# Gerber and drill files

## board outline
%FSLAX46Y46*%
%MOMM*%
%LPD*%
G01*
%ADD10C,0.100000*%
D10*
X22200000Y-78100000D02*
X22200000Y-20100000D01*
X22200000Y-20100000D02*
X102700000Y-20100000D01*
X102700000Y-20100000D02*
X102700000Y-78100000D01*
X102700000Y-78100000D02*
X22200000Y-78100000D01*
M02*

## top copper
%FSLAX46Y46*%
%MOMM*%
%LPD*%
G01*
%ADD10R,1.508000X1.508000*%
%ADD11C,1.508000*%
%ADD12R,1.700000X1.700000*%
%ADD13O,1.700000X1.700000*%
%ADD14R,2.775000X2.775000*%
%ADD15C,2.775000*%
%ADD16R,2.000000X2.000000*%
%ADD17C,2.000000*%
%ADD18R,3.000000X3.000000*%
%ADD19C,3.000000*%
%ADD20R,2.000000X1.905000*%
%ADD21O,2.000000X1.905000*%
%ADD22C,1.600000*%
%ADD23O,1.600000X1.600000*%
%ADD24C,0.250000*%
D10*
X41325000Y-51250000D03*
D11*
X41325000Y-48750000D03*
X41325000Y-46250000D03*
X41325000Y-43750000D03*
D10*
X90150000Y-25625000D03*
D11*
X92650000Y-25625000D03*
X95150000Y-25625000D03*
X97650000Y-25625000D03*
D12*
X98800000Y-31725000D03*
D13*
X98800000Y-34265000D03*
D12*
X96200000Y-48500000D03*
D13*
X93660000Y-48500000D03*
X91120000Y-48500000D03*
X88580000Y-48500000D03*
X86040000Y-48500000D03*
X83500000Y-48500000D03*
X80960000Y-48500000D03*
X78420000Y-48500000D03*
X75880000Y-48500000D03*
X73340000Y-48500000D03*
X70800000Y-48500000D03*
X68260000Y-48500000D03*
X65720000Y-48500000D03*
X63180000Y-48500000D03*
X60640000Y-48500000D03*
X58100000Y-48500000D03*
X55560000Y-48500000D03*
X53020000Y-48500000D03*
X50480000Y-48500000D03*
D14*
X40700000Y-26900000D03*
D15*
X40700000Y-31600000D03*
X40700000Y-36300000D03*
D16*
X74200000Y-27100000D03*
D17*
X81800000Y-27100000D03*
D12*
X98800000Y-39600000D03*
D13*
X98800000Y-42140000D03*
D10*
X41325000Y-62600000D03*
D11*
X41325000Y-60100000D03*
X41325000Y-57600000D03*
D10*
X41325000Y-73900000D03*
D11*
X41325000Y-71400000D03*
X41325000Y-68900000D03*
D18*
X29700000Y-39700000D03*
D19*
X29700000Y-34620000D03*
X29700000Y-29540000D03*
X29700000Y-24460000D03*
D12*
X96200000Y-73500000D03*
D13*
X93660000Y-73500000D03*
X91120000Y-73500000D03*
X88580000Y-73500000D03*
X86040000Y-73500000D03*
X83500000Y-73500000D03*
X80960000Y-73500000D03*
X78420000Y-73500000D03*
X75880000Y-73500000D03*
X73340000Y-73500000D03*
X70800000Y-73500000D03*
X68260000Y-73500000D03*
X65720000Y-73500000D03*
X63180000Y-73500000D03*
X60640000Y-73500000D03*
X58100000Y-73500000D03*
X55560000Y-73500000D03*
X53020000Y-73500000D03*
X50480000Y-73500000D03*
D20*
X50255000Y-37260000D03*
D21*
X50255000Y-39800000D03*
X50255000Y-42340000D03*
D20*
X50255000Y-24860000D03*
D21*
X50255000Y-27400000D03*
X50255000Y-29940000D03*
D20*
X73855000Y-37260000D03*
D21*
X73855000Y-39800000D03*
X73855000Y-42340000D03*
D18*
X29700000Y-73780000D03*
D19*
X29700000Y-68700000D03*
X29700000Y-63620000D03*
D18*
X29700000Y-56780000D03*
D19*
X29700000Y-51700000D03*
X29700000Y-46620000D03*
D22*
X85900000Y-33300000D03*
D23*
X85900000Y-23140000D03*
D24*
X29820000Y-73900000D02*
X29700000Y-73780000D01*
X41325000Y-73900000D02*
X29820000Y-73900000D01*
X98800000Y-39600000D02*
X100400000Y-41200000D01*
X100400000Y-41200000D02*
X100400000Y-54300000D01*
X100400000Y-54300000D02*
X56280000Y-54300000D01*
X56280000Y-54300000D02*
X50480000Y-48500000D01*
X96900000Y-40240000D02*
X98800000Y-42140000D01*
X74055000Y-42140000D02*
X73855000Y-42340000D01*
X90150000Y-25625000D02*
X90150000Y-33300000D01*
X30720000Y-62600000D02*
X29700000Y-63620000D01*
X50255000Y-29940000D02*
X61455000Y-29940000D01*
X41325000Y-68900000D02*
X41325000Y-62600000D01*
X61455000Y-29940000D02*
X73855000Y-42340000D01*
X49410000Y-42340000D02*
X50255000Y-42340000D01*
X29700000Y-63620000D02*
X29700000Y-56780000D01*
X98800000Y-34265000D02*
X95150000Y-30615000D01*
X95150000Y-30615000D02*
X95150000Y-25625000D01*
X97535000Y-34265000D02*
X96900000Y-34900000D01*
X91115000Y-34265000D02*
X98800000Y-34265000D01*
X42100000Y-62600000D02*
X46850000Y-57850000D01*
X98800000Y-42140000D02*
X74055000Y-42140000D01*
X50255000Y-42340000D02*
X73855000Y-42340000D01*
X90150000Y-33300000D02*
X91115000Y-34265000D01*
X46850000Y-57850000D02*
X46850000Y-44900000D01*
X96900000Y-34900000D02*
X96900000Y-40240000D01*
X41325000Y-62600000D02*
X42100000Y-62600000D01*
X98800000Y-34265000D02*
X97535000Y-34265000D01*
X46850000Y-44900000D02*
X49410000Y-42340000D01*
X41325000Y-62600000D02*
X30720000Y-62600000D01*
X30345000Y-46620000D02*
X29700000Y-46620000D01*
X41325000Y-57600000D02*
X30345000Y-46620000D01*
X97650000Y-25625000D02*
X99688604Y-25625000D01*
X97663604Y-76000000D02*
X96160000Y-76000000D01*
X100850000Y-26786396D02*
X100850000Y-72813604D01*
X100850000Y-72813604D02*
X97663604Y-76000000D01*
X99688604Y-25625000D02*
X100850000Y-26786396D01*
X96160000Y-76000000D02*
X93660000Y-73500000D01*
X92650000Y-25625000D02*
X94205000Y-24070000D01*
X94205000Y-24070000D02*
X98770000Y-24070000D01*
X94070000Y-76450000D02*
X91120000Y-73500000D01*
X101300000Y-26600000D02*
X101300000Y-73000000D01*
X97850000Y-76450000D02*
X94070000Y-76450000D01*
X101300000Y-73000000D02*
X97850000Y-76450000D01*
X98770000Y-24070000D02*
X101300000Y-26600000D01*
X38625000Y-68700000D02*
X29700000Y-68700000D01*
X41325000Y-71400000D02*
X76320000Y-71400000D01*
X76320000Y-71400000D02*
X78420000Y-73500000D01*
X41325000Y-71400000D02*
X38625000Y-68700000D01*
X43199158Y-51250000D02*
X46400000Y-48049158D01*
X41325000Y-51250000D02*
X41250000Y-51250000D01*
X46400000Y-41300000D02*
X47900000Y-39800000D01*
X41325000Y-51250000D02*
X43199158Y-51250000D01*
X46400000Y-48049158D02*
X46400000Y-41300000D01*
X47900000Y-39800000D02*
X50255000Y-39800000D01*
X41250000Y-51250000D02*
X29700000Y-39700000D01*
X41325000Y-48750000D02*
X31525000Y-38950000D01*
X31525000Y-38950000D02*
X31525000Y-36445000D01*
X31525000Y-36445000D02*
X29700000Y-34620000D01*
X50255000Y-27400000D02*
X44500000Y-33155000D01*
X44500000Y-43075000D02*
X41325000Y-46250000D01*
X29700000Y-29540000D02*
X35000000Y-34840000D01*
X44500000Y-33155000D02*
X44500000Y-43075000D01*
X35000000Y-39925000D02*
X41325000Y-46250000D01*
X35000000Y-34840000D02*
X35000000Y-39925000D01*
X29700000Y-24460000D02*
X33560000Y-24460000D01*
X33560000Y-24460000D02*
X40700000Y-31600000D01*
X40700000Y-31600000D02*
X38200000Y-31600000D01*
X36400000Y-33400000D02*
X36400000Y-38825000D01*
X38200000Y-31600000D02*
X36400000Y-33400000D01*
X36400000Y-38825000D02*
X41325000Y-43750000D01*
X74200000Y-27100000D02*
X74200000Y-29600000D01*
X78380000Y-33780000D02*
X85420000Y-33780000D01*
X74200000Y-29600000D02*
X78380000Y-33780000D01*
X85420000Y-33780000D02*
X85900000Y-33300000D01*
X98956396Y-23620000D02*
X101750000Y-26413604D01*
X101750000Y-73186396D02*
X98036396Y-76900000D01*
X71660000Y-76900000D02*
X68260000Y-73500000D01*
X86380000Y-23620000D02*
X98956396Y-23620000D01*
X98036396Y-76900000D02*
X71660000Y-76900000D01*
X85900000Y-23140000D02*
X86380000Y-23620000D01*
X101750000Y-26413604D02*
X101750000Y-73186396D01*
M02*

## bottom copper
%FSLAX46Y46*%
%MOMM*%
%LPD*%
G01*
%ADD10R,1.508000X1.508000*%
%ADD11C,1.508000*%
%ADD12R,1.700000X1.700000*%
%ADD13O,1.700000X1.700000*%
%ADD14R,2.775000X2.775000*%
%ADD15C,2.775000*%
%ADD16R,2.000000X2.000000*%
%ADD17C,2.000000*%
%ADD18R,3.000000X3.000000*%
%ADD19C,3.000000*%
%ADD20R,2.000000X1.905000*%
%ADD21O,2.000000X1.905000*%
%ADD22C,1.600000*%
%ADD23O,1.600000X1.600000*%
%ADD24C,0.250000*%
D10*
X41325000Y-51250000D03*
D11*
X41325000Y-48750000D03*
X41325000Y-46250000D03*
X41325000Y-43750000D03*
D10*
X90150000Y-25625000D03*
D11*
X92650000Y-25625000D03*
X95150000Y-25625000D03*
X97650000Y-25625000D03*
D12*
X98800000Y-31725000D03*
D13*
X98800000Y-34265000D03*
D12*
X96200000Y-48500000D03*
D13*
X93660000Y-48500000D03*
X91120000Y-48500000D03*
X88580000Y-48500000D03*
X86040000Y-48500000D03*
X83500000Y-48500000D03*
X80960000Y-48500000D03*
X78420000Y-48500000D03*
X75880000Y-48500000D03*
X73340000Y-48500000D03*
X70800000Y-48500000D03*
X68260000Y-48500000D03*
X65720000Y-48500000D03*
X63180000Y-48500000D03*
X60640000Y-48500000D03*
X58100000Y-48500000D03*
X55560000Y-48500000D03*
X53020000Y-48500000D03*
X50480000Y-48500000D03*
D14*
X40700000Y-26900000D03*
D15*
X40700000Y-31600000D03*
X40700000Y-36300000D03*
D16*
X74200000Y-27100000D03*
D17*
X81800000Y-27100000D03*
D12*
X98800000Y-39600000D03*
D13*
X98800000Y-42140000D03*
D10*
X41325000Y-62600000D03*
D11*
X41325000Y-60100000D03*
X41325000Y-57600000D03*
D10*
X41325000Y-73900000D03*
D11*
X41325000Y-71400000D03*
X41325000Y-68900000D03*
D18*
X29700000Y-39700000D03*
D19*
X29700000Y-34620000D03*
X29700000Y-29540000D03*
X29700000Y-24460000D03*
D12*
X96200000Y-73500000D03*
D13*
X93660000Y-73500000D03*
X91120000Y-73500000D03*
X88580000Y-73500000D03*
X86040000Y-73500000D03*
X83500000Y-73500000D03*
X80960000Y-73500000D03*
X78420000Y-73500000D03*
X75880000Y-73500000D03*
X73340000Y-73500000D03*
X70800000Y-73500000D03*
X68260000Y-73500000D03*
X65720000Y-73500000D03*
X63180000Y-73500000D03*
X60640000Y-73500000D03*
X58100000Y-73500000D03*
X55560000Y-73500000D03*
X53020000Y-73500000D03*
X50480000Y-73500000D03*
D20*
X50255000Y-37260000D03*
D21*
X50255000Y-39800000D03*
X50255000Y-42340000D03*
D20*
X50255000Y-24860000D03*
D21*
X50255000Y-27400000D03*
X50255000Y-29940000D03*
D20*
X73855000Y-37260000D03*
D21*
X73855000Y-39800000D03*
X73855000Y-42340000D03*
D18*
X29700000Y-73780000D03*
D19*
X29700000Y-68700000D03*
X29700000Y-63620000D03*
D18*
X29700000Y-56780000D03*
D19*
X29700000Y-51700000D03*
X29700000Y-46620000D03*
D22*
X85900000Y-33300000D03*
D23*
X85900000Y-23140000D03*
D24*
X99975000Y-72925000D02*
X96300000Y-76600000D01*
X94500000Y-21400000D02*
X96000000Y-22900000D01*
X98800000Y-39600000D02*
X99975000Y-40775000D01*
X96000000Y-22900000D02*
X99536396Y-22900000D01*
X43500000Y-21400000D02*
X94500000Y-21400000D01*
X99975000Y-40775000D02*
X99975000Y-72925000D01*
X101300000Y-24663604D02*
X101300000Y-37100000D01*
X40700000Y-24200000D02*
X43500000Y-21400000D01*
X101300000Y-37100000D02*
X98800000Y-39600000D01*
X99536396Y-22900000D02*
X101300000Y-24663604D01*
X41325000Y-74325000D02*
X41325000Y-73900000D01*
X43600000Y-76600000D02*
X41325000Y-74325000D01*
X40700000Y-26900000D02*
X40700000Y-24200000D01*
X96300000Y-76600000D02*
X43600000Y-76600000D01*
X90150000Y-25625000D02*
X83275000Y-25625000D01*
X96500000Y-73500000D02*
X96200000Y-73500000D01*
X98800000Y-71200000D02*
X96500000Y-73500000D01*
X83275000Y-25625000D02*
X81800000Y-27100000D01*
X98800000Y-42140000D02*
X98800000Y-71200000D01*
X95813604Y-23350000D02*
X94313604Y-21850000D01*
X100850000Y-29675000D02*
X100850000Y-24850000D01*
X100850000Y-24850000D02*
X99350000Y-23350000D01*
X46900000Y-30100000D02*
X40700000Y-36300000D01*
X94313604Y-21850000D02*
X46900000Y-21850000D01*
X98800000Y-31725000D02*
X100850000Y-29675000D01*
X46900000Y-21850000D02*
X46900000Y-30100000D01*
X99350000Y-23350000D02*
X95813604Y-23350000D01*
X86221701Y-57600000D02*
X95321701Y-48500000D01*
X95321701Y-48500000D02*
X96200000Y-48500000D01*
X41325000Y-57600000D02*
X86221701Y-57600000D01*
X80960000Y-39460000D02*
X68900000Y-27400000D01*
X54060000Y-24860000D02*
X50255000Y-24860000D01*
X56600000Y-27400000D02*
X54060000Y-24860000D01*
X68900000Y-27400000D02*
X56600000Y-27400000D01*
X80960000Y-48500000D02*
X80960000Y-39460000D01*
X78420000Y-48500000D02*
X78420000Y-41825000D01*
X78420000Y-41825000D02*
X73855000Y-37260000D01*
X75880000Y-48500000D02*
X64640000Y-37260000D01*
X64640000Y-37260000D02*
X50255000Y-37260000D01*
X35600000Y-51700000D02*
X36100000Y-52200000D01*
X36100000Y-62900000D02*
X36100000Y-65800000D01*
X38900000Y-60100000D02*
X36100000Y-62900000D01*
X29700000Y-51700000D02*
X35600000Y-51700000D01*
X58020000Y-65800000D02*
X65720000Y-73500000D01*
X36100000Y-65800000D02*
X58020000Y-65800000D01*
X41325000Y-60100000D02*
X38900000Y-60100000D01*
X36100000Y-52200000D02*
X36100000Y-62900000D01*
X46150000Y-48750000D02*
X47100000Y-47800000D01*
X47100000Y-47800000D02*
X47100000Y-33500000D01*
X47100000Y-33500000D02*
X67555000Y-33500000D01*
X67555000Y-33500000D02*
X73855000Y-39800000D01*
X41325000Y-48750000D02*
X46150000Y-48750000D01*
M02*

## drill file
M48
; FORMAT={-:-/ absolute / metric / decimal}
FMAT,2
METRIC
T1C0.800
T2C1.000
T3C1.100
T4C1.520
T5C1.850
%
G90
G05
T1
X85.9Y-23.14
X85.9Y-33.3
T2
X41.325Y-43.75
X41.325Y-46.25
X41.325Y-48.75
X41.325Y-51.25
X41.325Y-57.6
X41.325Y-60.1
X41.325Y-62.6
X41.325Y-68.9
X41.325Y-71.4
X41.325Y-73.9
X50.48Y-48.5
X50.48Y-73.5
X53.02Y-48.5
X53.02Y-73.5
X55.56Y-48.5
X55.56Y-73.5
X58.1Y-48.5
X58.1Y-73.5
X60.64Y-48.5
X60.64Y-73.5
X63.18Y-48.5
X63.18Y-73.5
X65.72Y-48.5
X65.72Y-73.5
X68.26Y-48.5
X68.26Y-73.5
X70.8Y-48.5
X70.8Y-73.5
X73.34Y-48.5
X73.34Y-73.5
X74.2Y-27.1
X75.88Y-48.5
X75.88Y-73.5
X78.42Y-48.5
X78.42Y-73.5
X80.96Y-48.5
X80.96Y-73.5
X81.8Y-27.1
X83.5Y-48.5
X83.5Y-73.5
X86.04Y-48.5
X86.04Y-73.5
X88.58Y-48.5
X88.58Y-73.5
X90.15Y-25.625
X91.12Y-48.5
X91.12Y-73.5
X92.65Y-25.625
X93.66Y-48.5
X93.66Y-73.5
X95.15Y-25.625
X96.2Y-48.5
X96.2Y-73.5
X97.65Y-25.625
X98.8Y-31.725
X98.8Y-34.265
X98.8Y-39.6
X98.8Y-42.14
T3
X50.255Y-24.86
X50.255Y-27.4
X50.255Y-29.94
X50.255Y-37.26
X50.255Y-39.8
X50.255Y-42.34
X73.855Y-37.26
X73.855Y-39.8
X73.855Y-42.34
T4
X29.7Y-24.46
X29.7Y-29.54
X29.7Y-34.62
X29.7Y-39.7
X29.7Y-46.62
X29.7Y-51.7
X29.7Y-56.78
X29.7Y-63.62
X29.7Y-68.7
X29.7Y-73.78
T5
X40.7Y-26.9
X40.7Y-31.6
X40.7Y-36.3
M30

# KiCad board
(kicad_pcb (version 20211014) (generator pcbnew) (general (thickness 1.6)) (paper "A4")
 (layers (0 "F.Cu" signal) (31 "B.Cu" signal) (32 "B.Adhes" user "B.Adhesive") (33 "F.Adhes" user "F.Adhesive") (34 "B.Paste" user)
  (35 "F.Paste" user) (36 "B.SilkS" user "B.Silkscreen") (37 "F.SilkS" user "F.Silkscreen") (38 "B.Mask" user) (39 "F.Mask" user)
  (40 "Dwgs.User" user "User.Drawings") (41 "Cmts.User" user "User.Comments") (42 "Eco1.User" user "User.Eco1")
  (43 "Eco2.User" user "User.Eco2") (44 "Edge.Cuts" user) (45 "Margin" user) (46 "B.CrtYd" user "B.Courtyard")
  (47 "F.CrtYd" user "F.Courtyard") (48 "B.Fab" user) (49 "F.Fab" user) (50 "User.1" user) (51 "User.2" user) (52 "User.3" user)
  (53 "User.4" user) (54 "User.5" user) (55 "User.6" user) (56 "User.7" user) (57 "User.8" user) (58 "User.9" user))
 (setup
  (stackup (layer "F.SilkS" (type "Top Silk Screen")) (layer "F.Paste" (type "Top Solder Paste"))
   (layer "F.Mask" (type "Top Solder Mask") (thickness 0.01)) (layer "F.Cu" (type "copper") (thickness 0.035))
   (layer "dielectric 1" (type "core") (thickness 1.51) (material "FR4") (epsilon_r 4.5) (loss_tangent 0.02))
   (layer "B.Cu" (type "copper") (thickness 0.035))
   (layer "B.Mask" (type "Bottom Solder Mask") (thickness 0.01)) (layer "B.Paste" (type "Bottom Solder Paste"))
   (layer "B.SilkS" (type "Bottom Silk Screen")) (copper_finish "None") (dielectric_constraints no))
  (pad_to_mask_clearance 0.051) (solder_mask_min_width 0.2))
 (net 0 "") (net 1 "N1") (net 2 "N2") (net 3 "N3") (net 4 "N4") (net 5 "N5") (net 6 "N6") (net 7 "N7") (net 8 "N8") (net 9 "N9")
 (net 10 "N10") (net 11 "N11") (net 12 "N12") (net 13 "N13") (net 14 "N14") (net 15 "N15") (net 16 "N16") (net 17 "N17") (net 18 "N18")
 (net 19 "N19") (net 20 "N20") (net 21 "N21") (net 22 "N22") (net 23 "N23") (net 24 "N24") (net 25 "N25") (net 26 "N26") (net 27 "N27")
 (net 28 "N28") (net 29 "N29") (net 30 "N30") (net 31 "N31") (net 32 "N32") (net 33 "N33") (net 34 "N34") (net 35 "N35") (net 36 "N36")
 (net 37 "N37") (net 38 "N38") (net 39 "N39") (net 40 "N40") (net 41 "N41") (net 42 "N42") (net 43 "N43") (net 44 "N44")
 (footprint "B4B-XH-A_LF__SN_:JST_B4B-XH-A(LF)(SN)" (layer "F.Cu") (at 40.8 47.5 90)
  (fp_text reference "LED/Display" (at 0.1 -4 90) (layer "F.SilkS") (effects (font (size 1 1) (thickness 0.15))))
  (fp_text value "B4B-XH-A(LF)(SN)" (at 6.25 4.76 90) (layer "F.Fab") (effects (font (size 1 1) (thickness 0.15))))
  (pad "1" thru_hole rect locked (at -3.75 0.525 90) (size 1.508 1.508) (drill 1) (layers *.Cu *.Mask) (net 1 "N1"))
  (pad "2" thru_hole circle locked (at -1.25 0.525 90) (size 1.508 1.508) (drill 1) (layers *.Cu *.Mask) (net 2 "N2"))
  (pad "3" thru_hole circle locked (at 1.25 0.525 90) (size 1.508 1.508) (drill 1) (layers *.Cu *.Mask) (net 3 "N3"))
  (pad "4" thru_hole circle locked (at 3.75 0.525 90) (size 1.508 1.508) (drill 1) (layers *.Cu *.Mask) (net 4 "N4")))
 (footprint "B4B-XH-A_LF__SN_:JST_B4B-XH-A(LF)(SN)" (layer "F.Cu") (at 93.9 25.1)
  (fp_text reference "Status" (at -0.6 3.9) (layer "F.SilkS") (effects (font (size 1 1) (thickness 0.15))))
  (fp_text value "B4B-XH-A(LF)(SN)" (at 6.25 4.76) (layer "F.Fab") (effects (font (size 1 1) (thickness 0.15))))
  (pad "1" thru_hole rect locked (at -3.75 0.525) (size 1.508 1.508) (drill 1) (layers *.Cu *.Mask) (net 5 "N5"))
  (pad "2" thru_hole circle locked (at -1.25 0.525) (size 1.508 1.508) (drill 1) (layers *.Cu *.Mask) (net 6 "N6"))
  (pad "3" thru_hole circle locked (at 1.25 0.525) (size 1.508 1.508) (drill 1) (layers *.Cu *.Mask) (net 5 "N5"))
  (pad "4" thru_hole circle locked (at 3.75 0.525) (size 1.508 1.508) (drill 1) (layers *.Cu *.Mask) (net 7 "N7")))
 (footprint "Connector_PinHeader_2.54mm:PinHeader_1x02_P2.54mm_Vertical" (layer "F.Cu") (at 98.8 31.725)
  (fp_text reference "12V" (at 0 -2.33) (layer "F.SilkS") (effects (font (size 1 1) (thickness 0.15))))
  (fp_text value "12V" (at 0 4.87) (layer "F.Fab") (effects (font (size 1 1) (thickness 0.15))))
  (pad "1" thru_hole rect (at 0 0) (size 1.7 1.7) (drill 1) (layers *.Cu *.Mask) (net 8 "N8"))
  (pad "2" thru_hole oval (at 0 2.54) (size 1.7 1.7) (drill 1) (layers *.Cu *.Mask) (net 5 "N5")))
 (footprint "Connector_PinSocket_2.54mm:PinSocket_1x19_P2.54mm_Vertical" (layer "F.Cu") (at 96.2 48.5 -90)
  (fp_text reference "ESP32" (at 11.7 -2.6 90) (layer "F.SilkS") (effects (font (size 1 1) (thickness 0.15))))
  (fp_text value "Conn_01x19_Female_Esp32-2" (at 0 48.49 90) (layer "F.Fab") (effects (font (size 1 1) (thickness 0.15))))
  (pad "1" thru_hole rect (at 0 0 270) (size 1.7 1.7) (drill 1) (layers *.Cu *.Mask) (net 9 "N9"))
  (pad "2" thru_hole oval (at 0 2.54 270) (size 1.7 1.7) (drill 1) (layers *.Cu *.Mask) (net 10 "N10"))
  (pad "3" thru_hole oval (at 0 5.08 270) (size 1.7 1.7) (drill 1) (layers *.Cu *.Mask) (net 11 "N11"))
  (pad "4" thru_hole oval (at 0 7.62 270) (size 1.7 1.7) (drill 1) (layers *.Cu *.Mask) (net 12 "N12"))
  (pad "5" thru_hole oval (at 0 10.16 270) (size 1.7 1.7) (drill 1) (layers *.Cu *.Mask) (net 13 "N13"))
  (pad "6" thru_hole oval (at 0 12.7 270) (size 1.7 1.7) (drill 1) (layers *.Cu *.Mask) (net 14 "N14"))
  (pad "7" thru_hole oval (at 0 15.24 270) (size 1.7 1.7) (drill 1) (layers *.Cu *.Mask) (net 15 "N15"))
  (pad "8" thru_hole oval (at 0 17.78 270) (size 1.7 1.7) (drill 1) (layers *.Cu *.Mask) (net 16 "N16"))
  (pad "9" thru_hole oval (at 0 20.32 270) (size 1.7 1.7) (drill 1) (layers *.Cu *.Mask) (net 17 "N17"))
  (pad "10" thru_hole oval (at 0 22.86 270) (size 1.7 1.7) (drill 1) (layers *.Cu *.Mask) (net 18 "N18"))
  (pad "11" thru_hole oval (at 0 25.4 270) (size 1.7 1.7) (drill 1) (layers *.Cu *.Mask) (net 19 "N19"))
  (pad "12" thru_hole oval (at 0 27.94 270) (size 1.7 1.7) (drill 1) (layers *.Cu *.Mask) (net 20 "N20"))
  (pad "13" thru_hole oval (at 0 30.48 270) (size 1.7 1.7) (drill 1) (layers *.Cu *.Mask) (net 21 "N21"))
  (pad "14" thru_hole oval (at 0 33.02 270) (size 1.7 1.7) (drill 1) (layers *.Cu *.Mask) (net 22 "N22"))
  (pad "15" thru_hole oval (at 0 35.56 270) (size 1.7 1.7) (drill 1) (layers *.Cu *.Mask) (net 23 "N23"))
  (pad "16" thru_hole oval (at 0 38.1 270) (size 1.7 1.7) (drill 1) (layers *.Cu *.Mask) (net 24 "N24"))
  (pad "17" thru_hole oval (at 0 40.64 270) (size 1.7 1.7) (drill 1) (layers *.Cu *.Mask) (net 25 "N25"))
  (pad "18" thru_hole oval (at 0 43.18 270) (size 1.7 1.7) (drill 1) (layers *.Cu *.Mask) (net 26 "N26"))
  (pad "19" thru_hole oval (at 0 45.72 270) (size 1.7 1.7) (drill 1) (layers *.Cu *.Mask) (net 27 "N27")))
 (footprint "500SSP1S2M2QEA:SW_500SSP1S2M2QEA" (layer "F.Cu") (at 40.7 31.6 -90)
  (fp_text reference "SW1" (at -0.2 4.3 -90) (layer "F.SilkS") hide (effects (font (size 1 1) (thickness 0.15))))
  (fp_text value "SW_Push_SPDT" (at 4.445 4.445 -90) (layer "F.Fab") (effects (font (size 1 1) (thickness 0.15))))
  (pad "1" thru_hole rect locked (at -4.7 0 270) (size 2.775 2.775) (drill 1.85) (layers *.Cu *.Mask) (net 27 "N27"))
  (pad "2" thru_hole circle locked (at 0 0 270) (size 2.775 2.775) (drill 1.85) (layers *.Cu *.Mask) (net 4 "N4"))
  (pad "3" thru_hole circle locked (at 4.7 0 270) (size 2.775 2.775) (drill 1.85) (layers *.Cu *.Mask) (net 8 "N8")))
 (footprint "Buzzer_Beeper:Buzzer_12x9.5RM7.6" (layer "F.Cu") (at 74.2 27.1)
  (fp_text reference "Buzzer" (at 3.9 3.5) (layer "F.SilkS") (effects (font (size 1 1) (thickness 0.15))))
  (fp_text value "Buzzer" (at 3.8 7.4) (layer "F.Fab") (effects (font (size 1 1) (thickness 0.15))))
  (pad "1" thru_hole rect (at 0 0) (size 2 2) (drill 1) (layers *.Cu *.Mask) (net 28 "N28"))
  (pad "2" thru_hole circle (at 7.6 0) (size 2 2) (drill 1) (layers *.Cu *.Mask) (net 5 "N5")))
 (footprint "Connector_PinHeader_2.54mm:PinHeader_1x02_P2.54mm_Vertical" (layer "F.Cu") (at 98.8 39.6)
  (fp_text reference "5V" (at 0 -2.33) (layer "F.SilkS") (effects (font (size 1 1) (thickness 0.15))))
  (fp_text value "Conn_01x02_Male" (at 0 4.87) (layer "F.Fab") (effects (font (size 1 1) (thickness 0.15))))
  (pad "1" thru_hole rect (at 0 0) (size 1.7 1.7) (drill 1) (layers *.Cu *.Mask) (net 27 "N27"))
  (pad "2" thru_hole oval (at 0 2.54) (size 1.7 1.7) (drill 1) (layers *.Cu *.Mask) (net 5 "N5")))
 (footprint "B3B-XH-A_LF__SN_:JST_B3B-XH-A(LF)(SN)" (layer "F.Cu") (at 40.8 60.1 90)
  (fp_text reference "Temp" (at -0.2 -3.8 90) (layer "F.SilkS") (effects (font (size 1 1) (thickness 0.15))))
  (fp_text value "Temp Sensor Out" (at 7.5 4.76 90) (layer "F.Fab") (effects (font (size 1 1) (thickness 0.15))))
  (pad "1" thru_hole rect locked (at -2.5 0.525 90) (size 1.508 1.508) (drill 1) (layers *.Cu *.Mask) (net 5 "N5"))
  (pad "2" thru_hole circle locked (at 0 0.525 90) (size 1.508 1.508) (drill 1) (layers *.Cu *.Mask) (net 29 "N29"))
  (pad "3" thru_hole circle locked (at 2.5 0.525 90) (size 1.508 1.508) (drill 1) (layers *.Cu *.Mask) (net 9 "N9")))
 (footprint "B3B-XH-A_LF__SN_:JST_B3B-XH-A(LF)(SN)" (layer "F.Cu") (at 40.8 71.4 90)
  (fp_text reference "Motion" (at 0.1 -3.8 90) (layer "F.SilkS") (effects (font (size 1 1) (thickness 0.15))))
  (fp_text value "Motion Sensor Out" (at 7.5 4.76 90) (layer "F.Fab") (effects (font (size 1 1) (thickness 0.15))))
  (pad "1" thru_hole rect locked (at -2.5 0.525 90) (size 1.508 1.508) (drill 1) (layers *.Cu *.Mask) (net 27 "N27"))
  (pad "2" thru_hole circle locked (at 0 0.525 90) (size 1.508 1.508) (drill 1) (layers *.Cu *.Mask) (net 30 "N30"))
  (pad "3" thru_hole circle locked (at 2.5 0.525 90) (size 1.508 1.508) (drill 1) (layers *.Cu *.Mask) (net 5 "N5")))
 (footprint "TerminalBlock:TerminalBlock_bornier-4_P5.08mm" (layer "F.Cu") (at 29.7 39.7 90)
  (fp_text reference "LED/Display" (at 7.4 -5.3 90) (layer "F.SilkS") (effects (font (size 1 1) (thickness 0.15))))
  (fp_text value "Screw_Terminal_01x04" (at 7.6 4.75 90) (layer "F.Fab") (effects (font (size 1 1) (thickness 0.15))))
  (pad "1" thru_hole rect (at 0 0 90) (size 3 3) (drill 1.52) (layers *.Cu *.Mask) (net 1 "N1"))
  (pad "2" thru_hole circle (at 5.08 0 90) (size 3 3) (drill 1.52) (layers *.Cu *.Mask) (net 2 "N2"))
  (pad "3" thru_hole circle (at 10.16 0 90) (size 3 3) (drill 1.52) (layers *.Cu *.Mask) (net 3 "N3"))
  (pad "4" thru_hole circle (at 15.24 0 90) (size 3 3) (drill 1.52) (layers *.Cu *.Mask) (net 4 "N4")))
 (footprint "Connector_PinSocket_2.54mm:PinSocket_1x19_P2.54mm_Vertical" (layer "F.Cu") (at 96.2 73.5 -90)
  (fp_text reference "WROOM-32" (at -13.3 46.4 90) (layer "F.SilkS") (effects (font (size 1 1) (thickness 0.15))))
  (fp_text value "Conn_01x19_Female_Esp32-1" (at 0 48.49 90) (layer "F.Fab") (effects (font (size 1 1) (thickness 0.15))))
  (pad "1" thru_hole rect (at 0 0 270) (size 1.7 1.7) (drill 1) (layers *.Cu *.Mask) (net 5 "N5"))
  (pad "2" thru_hole oval (at 0 2.54 270) (size 1.7 1.7) (drill 1) (layers *.Cu *.Mask) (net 7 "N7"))
  (pad "3" thru_hole oval (at 0 5.08 270) (size 1.7 1.7) (drill 1) (layers *.Cu *.Mask) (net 6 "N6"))
  (pad "4" thru_hole oval (at 0 7.62 270) (size 1.7 1.7) (drill 1) (layers *.Cu *.Mask) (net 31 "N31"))
  (pad "5" thru_hole oval (at 0 10.16 270) (size 1.7 1.7) (drill 1) (layers *.Cu *.Mask) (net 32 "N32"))
  (pad "6" thru_hole oval (at 0 12.7 270) (size 1.7 1.7) (drill 1) (layers *.Cu *.Mask) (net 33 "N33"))
  (pad "7" thru_hole oval (at 0 15.24 270) (size 1.7 1.7) (drill 1) (layers *.Cu *.Mask) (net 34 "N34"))
  (pad "8" thru_hole oval (at 0 17.78 270) (size 1.7 1.7) (drill 1) (layers *.Cu *.Mask) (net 30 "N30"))
  (pad "9" thru_hole oval (at 0 20.32 270) (size 1.7 1.7) (drill 1) (layers *.Cu *.Mask) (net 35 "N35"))
  (pad "10" thru_hole oval (at 0 22.86 270) (size 1.7 1.7) (drill 1) (layers *.Cu *.Mask) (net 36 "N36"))
  (pad "11" thru_hole oval (at 0 25.4 270) (size 1.7 1.7) (drill 1) (layers *.Cu *.Mask) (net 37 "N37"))
  (pad "12" thru_hole oval (at 0 27.94 270) (size 1.7 1.7) (drill 1) (layers *.Cu *.Mask) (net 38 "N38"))
  (pad "13" thru_hole oval (at 0 30.48 270) (size 1.7 1.7) (drill 1) (layers *.Cu *.Mask) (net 29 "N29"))
  (pad "14" thru_hole oval (at 0 33.02 270) (size 1.7 1.7) (drill 1) (layers *.Cu *.Mask) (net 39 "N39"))
  (pad "15" thru_hole oval (at 0 35.56 270) (size 1.7 1.7) (drill 1) (layers *.Cu *.Mask) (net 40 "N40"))
  (pad "16" thru_hole oval (at 0 38.1 270) (size 1.7 1.7) (drill 1) (layers *.Cu *.Mask) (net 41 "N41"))
  (pad "17" thru_hole oval (at 0 40.64 270) (size 1.7 1.7) (drill 1) (layers *.Cu *.Mask) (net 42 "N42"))
  (pad "18" thru_hole oval (at 0 43.18 270) (size 1.7 1.7) (drill 1) (layers *.Cu *.Mask) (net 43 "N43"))
  (pad "19" thru_hole oval (at 0 45.72 270) (size 1.7 1.7) (drill 1) (layers *.Cu *.Mask) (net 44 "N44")))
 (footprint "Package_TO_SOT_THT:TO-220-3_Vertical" (layer "F.Cu") (at 50.255 37.26 -90)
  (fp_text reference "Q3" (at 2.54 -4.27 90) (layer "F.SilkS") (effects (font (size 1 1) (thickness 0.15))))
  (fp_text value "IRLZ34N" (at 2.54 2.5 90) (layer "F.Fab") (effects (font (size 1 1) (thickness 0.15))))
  (pad "1" thru_hole rect (at 0 0 270) (size 1.905 2) (drill 1.1) (layers *.Cu *.Mask) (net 17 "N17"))
  (pad "2" thru_hole oval (at 2.54 0 270) (size 1.905 2) (drill 1.1) (layers *.Cu *.Mask) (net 1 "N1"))
  (pad "3" thru_hole oval (at 5.08 0 270) (size 1.905 2) (drill 1.1) (layers *.Cu *.Mask) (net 5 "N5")))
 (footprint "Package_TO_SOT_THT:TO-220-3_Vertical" (layer "F.Cu") (at 50.255 24.86 -90)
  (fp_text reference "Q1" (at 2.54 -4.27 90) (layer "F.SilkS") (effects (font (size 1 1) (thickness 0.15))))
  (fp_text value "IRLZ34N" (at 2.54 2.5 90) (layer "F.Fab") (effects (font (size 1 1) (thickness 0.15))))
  (pad "1" thru_hole rect (at 0 0 270) (size 1.905 2) (drill 1.1) (layers *.Cu *.Mask) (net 15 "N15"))
  (pad "2" thru_hole oval (at 2.54 0 270) (size 1.905 2) (drill 1.1) (layers *.Cu *.Mask) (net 3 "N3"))
  (pad "3" thru_hole oval (at 5.08 0 270) (size 1.905 2) (drill 1.1) (layers *.Cu *.Mask) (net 5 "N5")))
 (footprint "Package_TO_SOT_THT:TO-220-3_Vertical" (layer "F.Cu") (at 73.855 37.26 -90)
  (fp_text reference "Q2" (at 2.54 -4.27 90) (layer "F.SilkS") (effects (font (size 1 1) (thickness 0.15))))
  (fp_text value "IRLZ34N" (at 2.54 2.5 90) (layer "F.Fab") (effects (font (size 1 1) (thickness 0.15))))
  (pad "1" thru_hole rect (at 0 0 270) (size 1.905 2) (drill 1.1) (layers *.Cu *.Mask) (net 16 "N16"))
  (pad "2" thru_hole oval (at 2.54 0 270) (size 1.905 2) (drill 1.1) (layers *.Cu *.Mask) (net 2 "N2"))
  (pad "3" thru_hole oval (at 5.08 0 270) (size 1.905 2) (drill 1.1) (layers *.Cu *.Mask) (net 5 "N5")))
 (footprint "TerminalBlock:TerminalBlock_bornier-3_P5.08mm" (layer "F.Cu") (at 29.7 73.78 90)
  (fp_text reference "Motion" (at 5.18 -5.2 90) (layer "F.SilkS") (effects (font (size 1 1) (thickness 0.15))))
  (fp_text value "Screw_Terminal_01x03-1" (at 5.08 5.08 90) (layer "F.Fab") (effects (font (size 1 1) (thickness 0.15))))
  (pad "1" thru_hole rect (at 0 0 90) (size 3 3) (drill 1.52) (layers *.Cu *.Mask) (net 27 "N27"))
  (pad "2" thru_hole circle (at 5.08 0 90) (size 3 3) (drill 1.52) (layers *.Cu *.Mask) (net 30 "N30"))
  (pad "3" thru_hole circle (at 10.16 0 90) (size 3 3) (drill 1.52) (layers *.Cu *.Mask) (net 5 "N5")))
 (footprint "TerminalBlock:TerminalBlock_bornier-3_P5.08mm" (layer "F.Cu") (at 29.7 56.78 90)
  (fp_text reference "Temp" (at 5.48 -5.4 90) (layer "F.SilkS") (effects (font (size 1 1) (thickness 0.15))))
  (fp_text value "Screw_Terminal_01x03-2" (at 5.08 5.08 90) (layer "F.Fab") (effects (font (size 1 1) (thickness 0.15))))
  (pad "1" thru_hole rect (at 0 0 90) (size 3 3) (drill 1.52) (layers *.Cu *.Mask) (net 5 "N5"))
  (pad "2" thru_hole circle (at 5.08 0 90) (size 3 3) (drill 1.52) (layers *.Cu *.Mask) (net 29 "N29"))
  (pad "3" thru_hole circle (at 10.16 0 90) (size 3 3) (drill 1.52) (layers *.Cu *.Mask) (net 9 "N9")))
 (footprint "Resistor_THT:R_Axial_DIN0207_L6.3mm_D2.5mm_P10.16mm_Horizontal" (layer "F.Cu") (at 85.9 33.3 90)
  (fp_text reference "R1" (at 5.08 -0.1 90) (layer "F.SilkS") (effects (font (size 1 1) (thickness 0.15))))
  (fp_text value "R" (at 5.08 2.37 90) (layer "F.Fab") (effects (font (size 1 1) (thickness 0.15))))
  (pad "1" thru_hole circle (at 0 0 90) (size 1.6 1.6) (drill 0.8) (layers *.Cu *.Mask) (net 28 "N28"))
  (pad "2" thru_hole oval (at 10.16 0 90) (size 1.6 1.6) (drill 0.8) (layers *.Cu *.Mask) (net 38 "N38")))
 (gr_line (start 22.2 78.1) (end 22.2 20.1) (layer "Edge.Cuts") (width 0.1))
 (gr_line (start 22.2 20.1) (end 102.7 20.1) (layer "Edge.Cuts") (width 0.1))
 (gr_line (start 102.7 20.1) (end 102.7 78.1) (layer "Edge.Cuts") (width 0.1))
 (gr_line (start 102.7 78.1) (end 22.2 78.1) (layer "Edge.Cuts") (width 0.1))
 (segment (start 29.82 73.9) (end 29.7 73.78) (width 0.25) (layer "F.Cu") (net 27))
 (segment (start 41.325 73.9) (end 29.82 73.9) (width 0.25) (layer "F.Cu") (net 27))
 (segment (start 98.8 39.6) (end 100.4 41.2) (width 0.25) (layer "F.Cu") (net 27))
 (segment (start 100.4 41.2) (end 100.4 54.3) (width 0.25) (layer "F.Cu") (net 27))
 (segment (start 100.4 54.3) (end 56.28 54.3) (width 0.25) (layer "F.Cu") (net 27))
 (segment (start 56.28 54.3) (end 50.48 48.5) (width 0.25) (layer "F.Cu") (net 27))
 (segment (start 99.975 72.925) (end 96.3 76.6) (width 0.25) (layer "B.Cu") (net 27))
 (segment (start 94.5 21.4) (end 96 22.9) (width 0.25) (layer "B.Cu") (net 27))
 (segment (start 98.8 39.6) (end 99.975 40.775) (width 0.25) (layer "B.Cu") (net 27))
 (segment (start 96 22.9) (end 99.536396 22.9) (width 0.25) (layer "B.Cu") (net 27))
 (segment (start 43.5 21.4) (end 94.5 21.4) (width 0.25) (layer "B.Cu") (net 27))
 (segment (start 99.975 40.775) (end 99.975 72.925) (width 0.25) (layer "B.Cu") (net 27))
 (segment (start 101.3 24.663604) (end 101.3 37.1) (width 0.25) (layer "B.Cu") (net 27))
 (segment (start 40.7 24.2) (end 43.5 21.4) (width 0.25) (layer "B.Cu") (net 27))
 (segment (start 101.3 37.1) (end 98.8 39.6) (width 0.25) (layer "B.Cu") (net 27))
 (segment (start 99.536396 22.9) (end 101.3 24.663604) (width 0.25) (layer "B.Cu") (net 27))
 (segment (start 41.325 74.325) (end 41.325 73.9) (width 0.25) (layer "B.Cu") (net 27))
 (segment (start 43.6 76.6) (end 41.325 74.325) (width 0.25) (layer "B.Cu") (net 27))
 (segment (start 40.7 26.9) (end 40.7 24.2) (width 0.25) (layer "B.Cu") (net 27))
 (segment (start 96.3 76.6) (end 43.6 76.6) (width 0.25) (layer "B.Cu") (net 27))
 (segment (start 96.9 40.24) (end 98.8 42.14) (width 0.25) (layer "F.Cu") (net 5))
 (segment (start 74.055 42.14) (end 73.855 42.34) (width 0.25) (layer "F.Cu") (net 5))
 (segment (start 90.15 25.625) (end 90.15 33.3) (width 0.25) (layer "F.Cu") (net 5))
 (segment (start 30.72 62.6) (end 29.7 63.62) (width 0.25) (layer "F.Cu") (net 5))
 (segment (start 50.255 29.94) (end 61.455 29.94) (width 0.25) (layer "F.Cu") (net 5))
 (segment (start 41.325 68.9) (end 41.325 62.6) (width 0.25) (layer "F.Cu") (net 5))
 (segment (start 61.455 29.94) (end 73.855 42.34) (width 0.25) (layer "F.Cu") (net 5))
 (segment (start 49.41 42.34) (end 50.255 42.34) (width 0.25) (layer "F.Cu") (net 5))
 (segment (start 29.7 63.62) (end 29.7 56.78) (width 0.25) (layer "F.Cu") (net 5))
 (segment (start 98.8 34.265) (end 95.15 30.615) (width 0.25) (layer "F.Cu") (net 5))
 (segment (start 95.15 30.615) (end 95.15 25.625) (width 0.25) (layer "F.Cu") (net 5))
 (segment (start 97.535 34.265) (end 96.9 34.9) (width 0.25) (layer "F.Cu") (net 5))
 (segment (start 91.115 34.265) (end 98.8 34.265) (width 0.25) (layer "F.Cu") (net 5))
 (segment (start 42.1 62.6) (end 46.85 57.85) (width 0.25) (layer "F.Cu") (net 5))
 (segment (start 98.8 42.14) (end 74.055 42.14) (width 0.25) (layer "F.Cu") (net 5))
 (segment (start 50.255 42.34) (end 73.855 42.34) (width 0.25) (layer "F.Cu") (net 5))
 (segment (start 90.15 33.3) (end 91.115 34.265) (width 0.25) (layer "F.Cu") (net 5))
 (segment (start 46.85 57.85) (end 46.85 44.9) (width 0.25) (layer "F.Cu") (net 5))
 (segment (start 96.9 34.9) (end 96.9 40.24) (width 0.25) (layer "F.Cu") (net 5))
 (segment (start 41.325 62.6) (end 42.1 62.6) (width 0.25) (layer "F.Cu") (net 5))
 (segment (start 98.8 34.265) (end 97.535 34.265) (width 0.25) (layer "F.Cu") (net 5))
 (segment (start 46.85 44.9) (end 49.41 42.34) (width 0.25) (layer "F.Cu") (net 5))
 (segment (start 41.325 62.6) (end 30.72 62.6) (width 0.25) (layer "F.Cu") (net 5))
 (segment (start 90.15 25.625) (end 83.275 25.625) (width 0.25) (layer "B.Cu") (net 5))
 (segment (start 96.5 73.5) (end 96.2 73.5) (width 0.25) (layer "B.Cu") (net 5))
 (segment (start 98.8 71.2) (end 96.5 73.5) (width 0.25) (layer "B.Cu") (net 5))
 (segment (start 83.275 25.625) (end 81.8 27.1) (width 0.25) (layer "B.Cu") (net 5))
 (segment (start 98.8 42.14) (end 98.8 71.2) (width 0.25) (layer "B.Cu") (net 5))
 (segment (start 95.813604 23.35) (end 94.313604 21.85) (width 0.25) (layer "B.Cu") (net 8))
 (segment (start 100.85 29.675) (end 100.85 24.85) (width 0.25) (layer "B.Cu") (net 8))
 (segment (start 100.85 24.85) (end 99.35 23.35) (width 0.25) (layer "B.Cu") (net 8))
 (segment (start 46.9 30.1) (end 40.7 36.3) (width 0.25) (layer "B.Cu") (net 8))
 (segment (start 94.313604 21.85) (end 46.9 21.85) (width 0.25) (layer "B.Cu") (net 8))
 (segment (start 98.8 31.725) (end 100.85 29.675) (width 0.25) (layer "B.Cu") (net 8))
 (segment (start 46.9 21.85) (end 46.9 30.1) (width 0.25) (layer "B.Cu") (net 8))
 (segment (start 99.35 23.35) (end 95.813604 23.35) (width 0.25) (layer "B.Cu") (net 8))
 (segment (start 30.345 46.62) (end 29.7 46.62) (width 0.25) (layer "F.Cu") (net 9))
 (segment (start 41.325 57.6) (end 30.345 46.62) (width 0.25) (layer "F.Cu") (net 9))
 (segment (start 86.221701 57.6) (end 95.321701 48.5) (width 0.25) (layer "B.Cu") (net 9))
 (segment (start 95.321701 48.5) (end 96.2 48.5) (width 0.25) (layer "B.Cu") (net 9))
 (segment (start 41.325 57.6) (end 86.221701 57.6) (width 0.25) (layer "B.Cu") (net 9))
 (segment (start 97.65 25.625) (end 99.688604 25.625) (width 0.25) (layer "F.Cu") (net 7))
 (segment (start 97.663604 76) (end 96.16 76) (width 0.25) (layer "F.Cu") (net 7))
 (segment (start 100.85 26.786396) (end 100.85 72.813604) (width 0.25) (layer "F.Cu") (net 7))
 (segment (start 100.85 72.813604) (end 97.663604 76) (width 0.25) (layer "F.Cu") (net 7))
 (segment (start 99.688604 25.625) (end 100.85 26.786396) (width 0.25) (layer "F.Cu") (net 7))
 (segment (start 96.16 76) (end 93.66 73.5) (width 0.25) (layer "F.Cu") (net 7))
 (segment (start 92.65 25.625) (end 94.205 24.07) (width 0.25) (layer "F.Cu") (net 6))
 (segment (start 94.205 24.07) (end 98.77 24.07) (width 0.25) (layer "F.Cu") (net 6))
 (segment (start 94.07 76.45) (end 91.12 73.5) (width 0.25) (layer "F.Cu") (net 6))
 (segment (start 101.3 26.6) (end 101.3 73) (width 0.25) (layer "F.Cu") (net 6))
 (segment (start 97.85 76.45) (end 94.07 76.45) (width 0.25) (layer "F.Cu") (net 6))
 (segment (start 101.3 73) (end 97.85 76.45) (width 0.25) (layer "F.Cu") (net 6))
 (segment (start 98.77 24.07) (end 101.3 26.6) (width 0.25) (layer "F.Cu") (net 6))
 (segment (start 38.625 68.7) (end 29.7 68.7) (width 0.25) (layer "F.Cu") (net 30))
 (segment (start 41.325 71.4) (end 76.32 71.4) (width 0.25) (layer "F.Cu") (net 30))
 (segment (start 76.32 71.4) (end 78.42 73.5) (width 0.25) (layer "F.Cu") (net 30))
 (segment (start 41.325 71.4) (end 38.625 68.7) (width 0.25) (layer "F.Cu") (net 30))
 (segment (start 80.96 39.46) (end 68.9 27.4) (width 0.25) (layer "B.Cu") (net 15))
 (segment (start 54.06 24.86) (end 50.255 24.86) (width 0.25) (layer "B.Cu") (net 15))
 (segment (start 56.6 27.4) (end 54.06 24.86) (width 0.25) (layer "B.Cu") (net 15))
 (segment (start 68.9 27.4) (end 56.6 27.4) (width 0.25) (layer "B.Cu") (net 15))
 (segment (start 80.96 48.5) (end 80.96 39.46) (width 0.25) (layer "B.Cu") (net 15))
 (segment (start 78.42 48.5) (end 78.42 41.825) (width 0.25) (layer "B.Cu") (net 16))
 (segment (start 78.42 41.825) (end 73.855 37.26) (width 0.25) (layer "B.Cu") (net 16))
 (segment (start 75.88 48.5) (end 64.64 37.26) (width 0.25) (layer "B.Cu") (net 17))
 (segment (start 64.64 37.26) (end 50.255 37.26) (width 0.25) (layer "B.Cu") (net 17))
 (segment (start 43.199158 51.25) (end 46.4 48.049158) (width 0.25) (layer "F.Cu") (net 1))
 (segment (start 41.325 51.25) (end 41.25 51.25) (width 0.25) (layer "F.Cu") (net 1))
 (segment (start 46.4 41.3) (end 47.9 39.8) (width 0.25) (layer "F.Cu") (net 1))
 (segment (start 41.325 51.25) (end 43.199158 51.25) (width 0.25) (layer "F.Cu") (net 1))
 (segment (start 46.4 48.049158) (end 46.4 41.3) (width 0.25) (layer "F.Cu") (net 1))
 (segment (start 47.9 39.8) (end 50.255 39.8) (width 0.25) (layer "F.Cu") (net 1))
 (segment (start 41.25 51.25) (end 29.7 39.7) (width 0.25) (layer "F.Cu") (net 1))
 (segment (start 35.6 51.7) (end 36.1 52.2) (width 0.25) (layer "B.Cu") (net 29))
 (segment (start 36.1 62.9) (end 36.1 65.8) (width 0.25) (layer "B.Cu") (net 29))
 (segment (start 38.9 60.1) (end 36.1 62.9) (width 0.25) (layer "B.Cu") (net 29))
 (segment (start 29.7 51.7) (end 35.6 51.7) (width 0.25) (layer "B.Cu") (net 29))
 (segment (start 58.02 65.8) (end 65.72 73.5) (width 0.25) (layer "B.Cu") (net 29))
 (segment (start 36.1 65.8) (end 58.02 65.8) (width 0.25) (layer "B.Cu") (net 29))
 (segment (start 41.325 60.1) (end 38.9 60.1) (width 0.25) (layer "B.Cu") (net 29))
 (segment (start 36.1 52.2) (end 36.1 62.9) (width 0.25) (layer "B.Cu") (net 29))
 (segment (start 41.325 48.75) (end 31.525 38.95) (width 0.25) (layer "F.Cu") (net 2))
 (segment (start 31.525 38.95) (end 31.525 36.445) (width 0.25) (layer "F.Cu") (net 2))
 (segment (start 31.525 36.445) (end 29.7 34.62) (width 0.25) (layer "F.Cu") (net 2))
 (segment (start 46.15 48.75) (end 47.1 47.8) (width 0.25) (layer "B.Cu") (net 2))
 (segment (start 47.1 47.8) (end 47.1 33.5) (width 0.25) (layer "B.Cu") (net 2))
 (segment (start 47.1 33.5) (end 67.555 33.5) (width 0.25) (layer "B.Cu") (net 2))
 (segment (start 67.555 33.5) (end 73.855 39.8) (width 0.25) (layer "B.Cu") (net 2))
 (segment (start 41.325 48.75) (end 46.15 48.75) (width 0.25) (layer "B.Cu") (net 2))
 (segment (start 50.255 27.4) (end 44.5 33.155) (width 0.25) (layer "F.Cu") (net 3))
 (segment (start 44.5 43.075) (end 41.325 46.25) (width 0.25) (layer "F.Cu") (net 3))
 (segment (start 29.7 29.54) (end 35 34.84) (width 0.25) (layer "F.Cu") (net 3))
 (segment (start 44.5 33.155) (end 44.5 43.075) (width 0.25) (layer "F.Cu") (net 3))
 (segment (start 35 39.925) (end 41.325 46.25) (width 0.25) (layer "F.Cu") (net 3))
 (segment (start 35 34.84) (end 35 39.925) (width 0.25) (layer "F.Cu") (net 3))
 (segment (start 29.7 24.46) (end 33.56 24.46) (width 0.25) (layer "F.Cu") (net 4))
 (segment (start 33.56 24.46) (end 40.7 31.6) (width 0.25) (layer "F.Cu") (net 4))
 (segment (start 40.7 31.6) (end 38.2 31.6) (width 0.25) (layer "F.Cu") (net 4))
 (segment (start 36.4 33.4) (end 36.4 38.825) (width 0.25) (layer "F.Cu") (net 4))
 (segment (start 38.2 31.6) (end 36.4 33.4) (width 0.25) (layer "F.Cu") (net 4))
 (segment (start 36.4 38.825) (end 41.325 43.75) (width 0.25) (layer "F.Cu") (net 4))
 (segment (start 74.2 27.1) (end 74.2 29.6) (width 0.25) (layer "F.Cu") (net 28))
 (segment (start 78.38 33.78) (end 85.42 33.78) (width 0.25) (layer "F.Cu") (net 28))
 (segment (start 74.2 29.6) (end 78.38 33.78) (width 0.25) (layer "F.Cu") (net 28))
 (segment (start 85.42 33.78) (end 85.9 33.3) (width 0.25) (layer "F.Cu") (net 28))
 (segment (start 98.956396 23.62) (end 101.75 26.413604) (width 0.25) (layer "F.Cu") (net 38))
 (segment (start 101.75 73.186396) (end 98.036396 76.9) (width 0.25) (layer "F.Cu") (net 38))
 (segment (start 71.66 76.9) (end 68.26 73.5) (width 0.25) (layer "F.Cu") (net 38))
 (segment (start 86.38 23.62) (end 98.956396 23.62) (width 0.25) (layer "F.Cu") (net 38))
 (segment (start 98.036396 76.9) (end 71.66 76.9) (width 0.25) (layer "F.Cu") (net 38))
 (segment (start 85.9 23.14) (end 86.38 23.62) (width 0.25) (layer "F.Cu") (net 38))
 (segment (start 101.75 26.413604) (end 101.75 73.186396) (width 0.25) (layer "F.Cu") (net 38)))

